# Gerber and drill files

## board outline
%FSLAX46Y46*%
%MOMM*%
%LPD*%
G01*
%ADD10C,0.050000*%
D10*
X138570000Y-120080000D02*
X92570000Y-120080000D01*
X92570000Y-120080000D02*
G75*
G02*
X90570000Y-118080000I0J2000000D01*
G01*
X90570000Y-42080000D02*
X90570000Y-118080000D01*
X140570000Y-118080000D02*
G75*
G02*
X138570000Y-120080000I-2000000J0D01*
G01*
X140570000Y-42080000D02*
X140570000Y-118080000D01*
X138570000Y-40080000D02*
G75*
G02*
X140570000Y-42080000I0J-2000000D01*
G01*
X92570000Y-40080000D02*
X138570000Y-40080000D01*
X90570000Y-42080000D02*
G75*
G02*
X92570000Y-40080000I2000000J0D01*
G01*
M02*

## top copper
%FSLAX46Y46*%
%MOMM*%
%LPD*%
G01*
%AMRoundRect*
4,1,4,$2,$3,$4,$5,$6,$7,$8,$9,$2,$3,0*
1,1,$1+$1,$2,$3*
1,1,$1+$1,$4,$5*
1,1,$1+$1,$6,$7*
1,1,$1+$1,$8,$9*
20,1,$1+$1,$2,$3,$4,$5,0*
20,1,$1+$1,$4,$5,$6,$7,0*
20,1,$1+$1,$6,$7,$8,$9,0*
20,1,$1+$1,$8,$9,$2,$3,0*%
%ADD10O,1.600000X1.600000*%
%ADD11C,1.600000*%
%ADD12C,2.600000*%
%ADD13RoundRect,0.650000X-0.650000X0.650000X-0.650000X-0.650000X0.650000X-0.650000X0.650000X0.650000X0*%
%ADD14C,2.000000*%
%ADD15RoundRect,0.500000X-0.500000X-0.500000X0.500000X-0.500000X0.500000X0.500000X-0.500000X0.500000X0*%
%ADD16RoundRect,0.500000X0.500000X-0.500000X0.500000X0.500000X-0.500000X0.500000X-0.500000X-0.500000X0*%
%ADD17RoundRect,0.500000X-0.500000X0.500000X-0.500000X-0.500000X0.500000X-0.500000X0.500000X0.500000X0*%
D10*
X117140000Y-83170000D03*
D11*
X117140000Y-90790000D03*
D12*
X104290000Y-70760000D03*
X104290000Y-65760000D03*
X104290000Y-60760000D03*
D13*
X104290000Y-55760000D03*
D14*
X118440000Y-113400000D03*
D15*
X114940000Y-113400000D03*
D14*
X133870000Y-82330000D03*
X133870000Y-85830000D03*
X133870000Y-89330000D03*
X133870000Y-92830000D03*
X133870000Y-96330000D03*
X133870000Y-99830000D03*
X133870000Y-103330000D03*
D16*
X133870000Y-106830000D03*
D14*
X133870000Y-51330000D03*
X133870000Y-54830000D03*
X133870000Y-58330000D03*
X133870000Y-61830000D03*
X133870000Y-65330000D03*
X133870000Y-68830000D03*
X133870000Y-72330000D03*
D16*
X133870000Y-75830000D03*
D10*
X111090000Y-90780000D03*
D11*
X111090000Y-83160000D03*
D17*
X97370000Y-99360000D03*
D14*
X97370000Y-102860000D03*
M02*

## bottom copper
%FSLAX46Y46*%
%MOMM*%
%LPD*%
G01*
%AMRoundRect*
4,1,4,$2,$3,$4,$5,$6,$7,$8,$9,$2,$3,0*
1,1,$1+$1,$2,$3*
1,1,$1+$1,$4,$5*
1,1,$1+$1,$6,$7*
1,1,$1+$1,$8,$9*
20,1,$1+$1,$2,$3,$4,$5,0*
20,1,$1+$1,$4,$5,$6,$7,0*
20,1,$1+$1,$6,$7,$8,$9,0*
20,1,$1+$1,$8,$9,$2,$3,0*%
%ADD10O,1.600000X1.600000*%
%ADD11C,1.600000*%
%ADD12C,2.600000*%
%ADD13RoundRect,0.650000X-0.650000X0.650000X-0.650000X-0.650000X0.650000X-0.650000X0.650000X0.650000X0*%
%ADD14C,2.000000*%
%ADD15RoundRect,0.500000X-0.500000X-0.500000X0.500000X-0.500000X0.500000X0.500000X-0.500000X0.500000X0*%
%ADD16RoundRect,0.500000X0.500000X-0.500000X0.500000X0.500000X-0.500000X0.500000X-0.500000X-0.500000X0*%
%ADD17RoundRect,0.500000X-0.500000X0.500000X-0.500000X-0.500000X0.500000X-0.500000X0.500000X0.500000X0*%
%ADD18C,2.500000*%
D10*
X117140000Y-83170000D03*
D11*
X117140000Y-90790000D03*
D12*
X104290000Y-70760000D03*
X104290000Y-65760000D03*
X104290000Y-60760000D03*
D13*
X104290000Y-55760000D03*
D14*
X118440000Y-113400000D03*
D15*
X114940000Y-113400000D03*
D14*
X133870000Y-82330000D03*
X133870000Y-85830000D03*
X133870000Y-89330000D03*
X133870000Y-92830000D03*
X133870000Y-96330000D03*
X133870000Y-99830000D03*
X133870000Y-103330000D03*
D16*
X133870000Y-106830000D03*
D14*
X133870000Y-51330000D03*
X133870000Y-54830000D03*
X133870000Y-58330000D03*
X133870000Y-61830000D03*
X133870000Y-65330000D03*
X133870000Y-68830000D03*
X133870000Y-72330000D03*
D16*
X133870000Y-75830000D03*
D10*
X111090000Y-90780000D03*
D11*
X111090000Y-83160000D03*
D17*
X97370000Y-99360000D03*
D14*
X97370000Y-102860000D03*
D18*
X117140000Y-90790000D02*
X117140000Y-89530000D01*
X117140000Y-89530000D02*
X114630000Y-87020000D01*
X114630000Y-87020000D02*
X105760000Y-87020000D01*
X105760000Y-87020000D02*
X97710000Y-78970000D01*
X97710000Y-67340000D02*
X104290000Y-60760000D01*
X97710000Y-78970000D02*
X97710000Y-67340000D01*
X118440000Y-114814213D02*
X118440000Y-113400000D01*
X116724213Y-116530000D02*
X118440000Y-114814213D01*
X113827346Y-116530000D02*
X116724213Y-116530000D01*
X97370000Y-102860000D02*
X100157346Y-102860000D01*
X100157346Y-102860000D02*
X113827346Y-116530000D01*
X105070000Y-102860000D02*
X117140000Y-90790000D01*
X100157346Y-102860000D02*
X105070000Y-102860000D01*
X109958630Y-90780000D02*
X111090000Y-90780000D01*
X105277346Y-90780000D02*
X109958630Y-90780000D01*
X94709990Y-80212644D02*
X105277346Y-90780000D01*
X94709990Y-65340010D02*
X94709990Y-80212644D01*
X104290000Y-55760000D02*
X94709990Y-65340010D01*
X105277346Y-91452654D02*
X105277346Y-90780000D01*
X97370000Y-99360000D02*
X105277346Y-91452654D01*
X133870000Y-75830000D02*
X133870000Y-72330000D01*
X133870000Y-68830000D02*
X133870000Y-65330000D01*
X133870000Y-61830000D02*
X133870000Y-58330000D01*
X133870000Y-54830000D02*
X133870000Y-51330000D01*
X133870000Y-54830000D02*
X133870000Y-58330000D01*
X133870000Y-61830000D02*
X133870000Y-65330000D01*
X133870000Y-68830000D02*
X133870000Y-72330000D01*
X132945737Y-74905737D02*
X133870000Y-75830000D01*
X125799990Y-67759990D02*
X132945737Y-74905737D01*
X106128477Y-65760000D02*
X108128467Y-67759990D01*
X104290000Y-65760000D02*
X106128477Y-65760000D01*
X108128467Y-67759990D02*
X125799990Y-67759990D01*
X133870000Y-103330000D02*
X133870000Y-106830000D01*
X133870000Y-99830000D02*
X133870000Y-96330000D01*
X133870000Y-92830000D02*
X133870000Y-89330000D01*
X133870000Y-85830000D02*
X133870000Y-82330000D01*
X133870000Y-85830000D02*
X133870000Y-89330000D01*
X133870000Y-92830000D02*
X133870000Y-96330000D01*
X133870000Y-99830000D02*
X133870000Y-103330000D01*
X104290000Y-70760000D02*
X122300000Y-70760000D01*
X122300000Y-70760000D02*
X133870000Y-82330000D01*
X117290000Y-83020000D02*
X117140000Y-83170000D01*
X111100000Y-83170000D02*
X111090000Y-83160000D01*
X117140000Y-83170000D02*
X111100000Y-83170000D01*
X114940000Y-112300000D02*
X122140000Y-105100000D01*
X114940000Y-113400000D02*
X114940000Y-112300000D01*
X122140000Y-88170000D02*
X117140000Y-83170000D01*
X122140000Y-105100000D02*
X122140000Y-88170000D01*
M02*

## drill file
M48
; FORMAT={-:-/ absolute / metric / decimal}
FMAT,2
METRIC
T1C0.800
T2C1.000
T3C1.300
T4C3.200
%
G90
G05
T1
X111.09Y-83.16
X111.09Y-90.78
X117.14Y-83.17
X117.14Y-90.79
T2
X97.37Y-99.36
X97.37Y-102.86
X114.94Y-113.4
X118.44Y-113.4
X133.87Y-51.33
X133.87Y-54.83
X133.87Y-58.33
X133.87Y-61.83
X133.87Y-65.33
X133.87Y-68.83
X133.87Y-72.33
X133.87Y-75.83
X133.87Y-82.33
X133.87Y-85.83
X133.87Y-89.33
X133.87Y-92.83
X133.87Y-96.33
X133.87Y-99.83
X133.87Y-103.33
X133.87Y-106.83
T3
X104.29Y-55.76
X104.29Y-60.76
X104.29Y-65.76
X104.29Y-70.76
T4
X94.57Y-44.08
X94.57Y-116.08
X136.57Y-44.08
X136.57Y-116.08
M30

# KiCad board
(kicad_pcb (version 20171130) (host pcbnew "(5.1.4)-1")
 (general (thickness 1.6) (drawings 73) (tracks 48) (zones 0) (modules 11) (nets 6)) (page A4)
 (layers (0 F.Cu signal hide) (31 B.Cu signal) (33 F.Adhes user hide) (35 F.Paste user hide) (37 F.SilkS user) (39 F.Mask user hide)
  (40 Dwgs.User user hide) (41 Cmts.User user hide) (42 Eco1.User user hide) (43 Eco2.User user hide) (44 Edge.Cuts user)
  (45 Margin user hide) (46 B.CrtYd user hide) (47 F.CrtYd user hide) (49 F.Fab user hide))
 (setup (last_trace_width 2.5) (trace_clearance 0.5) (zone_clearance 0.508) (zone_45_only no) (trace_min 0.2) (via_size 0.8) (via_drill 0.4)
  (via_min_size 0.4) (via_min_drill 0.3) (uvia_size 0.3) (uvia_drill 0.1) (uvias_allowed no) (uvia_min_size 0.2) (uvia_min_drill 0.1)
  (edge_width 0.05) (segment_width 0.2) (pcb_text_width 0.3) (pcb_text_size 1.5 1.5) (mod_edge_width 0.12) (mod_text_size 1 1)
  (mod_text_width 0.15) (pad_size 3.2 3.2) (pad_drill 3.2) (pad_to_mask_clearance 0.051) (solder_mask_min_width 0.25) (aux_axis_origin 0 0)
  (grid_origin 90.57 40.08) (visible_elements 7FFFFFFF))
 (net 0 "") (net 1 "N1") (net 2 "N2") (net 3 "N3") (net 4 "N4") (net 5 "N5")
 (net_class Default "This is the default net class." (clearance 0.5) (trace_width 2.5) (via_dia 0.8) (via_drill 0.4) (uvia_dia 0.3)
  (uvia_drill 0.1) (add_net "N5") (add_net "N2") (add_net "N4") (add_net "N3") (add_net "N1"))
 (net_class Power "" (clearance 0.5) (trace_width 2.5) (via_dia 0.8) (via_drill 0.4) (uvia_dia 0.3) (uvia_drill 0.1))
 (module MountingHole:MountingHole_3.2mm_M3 (layer F.Cu) (at 94.57 116.08)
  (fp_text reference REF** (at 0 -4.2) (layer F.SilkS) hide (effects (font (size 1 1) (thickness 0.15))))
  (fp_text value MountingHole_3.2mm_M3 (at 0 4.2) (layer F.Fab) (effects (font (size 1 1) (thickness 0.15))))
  (pad 1 np_thru_hole circle (at 0 0) (size 3.2 3.2) (drill 3.2) (layers *.Cu *.Mask)))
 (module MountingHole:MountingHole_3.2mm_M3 (layer F.Cu) (at 136.57 116.08)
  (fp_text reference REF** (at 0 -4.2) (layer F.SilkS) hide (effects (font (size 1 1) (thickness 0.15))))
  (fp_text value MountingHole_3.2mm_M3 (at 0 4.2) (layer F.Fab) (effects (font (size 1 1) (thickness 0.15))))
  (pad 1 np_thru_hole circle (at 0 0) (size 3.2 3.2) (drill 3.2) (layers *.Cu *.Mask)))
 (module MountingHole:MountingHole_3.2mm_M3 (layer F.Cu) (at 136.57 44.08)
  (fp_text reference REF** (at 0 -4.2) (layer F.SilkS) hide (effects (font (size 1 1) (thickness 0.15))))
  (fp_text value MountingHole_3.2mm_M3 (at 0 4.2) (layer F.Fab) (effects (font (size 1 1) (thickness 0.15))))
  (pad 1 np_thru_hole circle (at 0 0) (size 3.2 3.2) (drill 3.2) (layers *.Cu *.Mask)))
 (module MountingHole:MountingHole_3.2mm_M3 (layer F.Cu) (at 94.57 44.08)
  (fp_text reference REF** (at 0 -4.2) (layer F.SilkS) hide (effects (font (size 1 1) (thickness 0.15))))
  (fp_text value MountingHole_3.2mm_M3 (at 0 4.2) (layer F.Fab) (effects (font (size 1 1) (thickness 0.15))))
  (pad 1 np_thru_hole circle (at 0 0) (size 3.2 3.2) (drill 3.2) (layers *.Cu *.Mask)))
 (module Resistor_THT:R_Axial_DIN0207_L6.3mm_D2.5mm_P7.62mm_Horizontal (layer F.Cu) (at 117.14 90.79 90)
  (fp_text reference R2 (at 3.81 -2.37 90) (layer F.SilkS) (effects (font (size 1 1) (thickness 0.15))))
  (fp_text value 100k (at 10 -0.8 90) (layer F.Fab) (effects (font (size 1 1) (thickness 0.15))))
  (pad 2 thru_hole oval (at 7.62 0 90) (size 1.6 1.6) (drill 0.8) (layers *.Cu *.Mask) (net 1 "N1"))
  (pad 1 thru_hole circle (at 0 0 90) (size 1.6 1.6) (drill 0.8) (layers *.Cu *.Mask) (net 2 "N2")))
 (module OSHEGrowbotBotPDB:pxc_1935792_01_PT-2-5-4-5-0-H (layer F.Cu) (at 99.79 53.26 270)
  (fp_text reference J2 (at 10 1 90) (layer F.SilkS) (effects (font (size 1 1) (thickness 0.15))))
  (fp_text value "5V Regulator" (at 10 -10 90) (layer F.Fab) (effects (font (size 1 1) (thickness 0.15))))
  (pad 4 thru_hole circle (at 17.5 -4.5 270) (size 2.6 2.6) (drill 1.3) (layers *.Cu *.Mask) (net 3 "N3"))
  (pad 3 thru_hole circle (at 12.5 -4.5 270) (size 2.6 2.6) (drill 1.3) (layers *.Cu *.Mask) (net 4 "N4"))
  (pad 2 thru_hole circle (at 7.5 -4.5 270) (size 2.6 2.6) (drill 1.3) (layers *.Cu *.Mask) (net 2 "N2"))
  (pad 1 thru_hole roundrect (at 2.5 -4.5 270) (size 2.6 2.6) (drill 1.3) (layers *.Cu *.Mask) (roundrect_rratio 0.25) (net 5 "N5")))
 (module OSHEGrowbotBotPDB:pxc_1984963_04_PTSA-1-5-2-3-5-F (layer F.Cu) (at 111.69 118.1)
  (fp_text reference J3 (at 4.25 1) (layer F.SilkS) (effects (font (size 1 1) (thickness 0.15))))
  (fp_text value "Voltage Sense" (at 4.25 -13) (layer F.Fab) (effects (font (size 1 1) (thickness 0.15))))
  (pad 2 thru_hole circle (at 6.75 -4.7) (size 2 2) (drill 1) (layers *.Cu *.Mask) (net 2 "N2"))
  (pad 1 thru_hole roundrect (at 3.25 -4.7) (size 2 2) (drill 1) (layers *.Cu *.Mask) (roundrect_rratio 0.25) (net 1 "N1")))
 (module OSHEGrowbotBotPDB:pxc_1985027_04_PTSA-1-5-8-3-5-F (layer F.Cu) (at 138.57 110.08 90)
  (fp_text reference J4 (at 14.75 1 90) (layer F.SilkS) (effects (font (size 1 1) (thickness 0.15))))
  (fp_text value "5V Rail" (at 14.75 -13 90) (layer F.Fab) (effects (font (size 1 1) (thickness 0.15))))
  (pad 8 thru_hole circle (at 27.75 -4.7 90) (size 2 2) (drill 1) (layers *.Cu *.Mask) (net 3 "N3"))
  (pad 7 thru_hole circle (at 24.25 -4.7 90) (size 2 2) (drill 1) (layers *.Cu *.Mask) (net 3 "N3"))
  (pad 6 thru_hole circle (at 20.75 -4.7 90) (size 2 2) (drill 1) (layers *.Cu *.Mask) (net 3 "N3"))
  (pad 5 thru_hole circle (at 17.25 -4.7 90) (size 2 2) (drill 1) (layers *.Cu *.Mask) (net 3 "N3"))
  (pad 4 thru_hole circle (at 13.75 -4.7 90) (size 2 2) (drill 1) (layers *.Cu *.Mask) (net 3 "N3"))
  (pad 3 thru_hole circle (at 10.25 -4.7 90) (size 2 2) (drill 1) (layers *.Cu *.Mask) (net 3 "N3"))
  (pad 2 thru_hole circle (at 6.75 -4.7 90) (size 2 2) (drill 1) (layers *.Cu *.Mask) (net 3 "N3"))
  (pad 1 thru_hole roundrect (at 3.25 -4.7 90) (size 2 2) (drill 1) (layers *.Cu *.Mask) (roundrect_rratio 0.25) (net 3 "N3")))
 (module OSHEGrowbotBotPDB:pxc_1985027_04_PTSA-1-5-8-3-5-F (layer F.Cu) (at 138.57 79.08 90)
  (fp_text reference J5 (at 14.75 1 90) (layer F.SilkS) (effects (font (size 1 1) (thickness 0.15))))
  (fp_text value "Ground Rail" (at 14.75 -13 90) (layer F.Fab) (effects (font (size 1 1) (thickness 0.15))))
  (pad 8 thru_hole circle (at 27.75 -4.7 90) (size 2 2) (drill 1) (layers *.Cu *.Mask) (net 4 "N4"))
  (pad 7 thru_hole circle (at 24.25 -4.7 90) (size 2 2) (drill 1) (layers *.Cu *.Mask) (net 4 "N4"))
  (pad 6 thru_hole circle (at 20.75 -4.7 90) (size 2 2) (drill 1) (layers *.Cu *.Mask) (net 4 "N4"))
  (pad 5 thru_hole circle (at 17.25 -4.7 90) (size 2 2) (drill 1) (layers *.Cu *.Mask) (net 4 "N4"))
  (pad 4 thru_hole circle (at 13.75 -4.7 90) (size 2 2) (drill 1) (layers *.Cu *.Mask) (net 4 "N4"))
  (pad 3 thru_hole circle (at 10.25 -4.7 90) (size 2 2) (drill 1) (layers *.Cu *.Mask) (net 4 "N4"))
  (pad 2 thru_hole circle (at 6.75 -4.7 90) (size 2 2) (drill 1) (layers *.Cu *.Mask) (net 4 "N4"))
  (pad 1 thru_hole roundrect (at 3.25 -4.7 90) (size 2 2) (drill 1) (layers *.Cu *.Mask) (roundrect_rratio 0.25) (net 4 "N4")))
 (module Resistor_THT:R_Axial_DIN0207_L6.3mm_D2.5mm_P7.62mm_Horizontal (layer F.Cu) (at 111.09 83.16 270)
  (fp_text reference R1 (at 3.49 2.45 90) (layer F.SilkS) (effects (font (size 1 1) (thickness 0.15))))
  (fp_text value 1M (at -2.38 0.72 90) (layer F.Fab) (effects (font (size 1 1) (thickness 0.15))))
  (pad 2 thru_hole oval (at 7.62 0 270) (size 1.6 1.6) (drill 0.8) (layers *.Cu *.Mask) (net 5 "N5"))
  (pad 1 thru_hole circle (at 0 0 270) (size 1.6 1.6) (drill 0.8) (layers *.Cu *.Mask) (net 1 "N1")))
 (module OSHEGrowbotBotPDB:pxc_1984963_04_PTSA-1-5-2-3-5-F (layer F.Cu) (at 92.67 96.11 270)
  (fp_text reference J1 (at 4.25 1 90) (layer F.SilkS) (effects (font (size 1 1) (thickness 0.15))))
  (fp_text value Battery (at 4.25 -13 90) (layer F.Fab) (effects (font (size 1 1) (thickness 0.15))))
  (pad 1 thru_hole roundrect (at 3.25 -4.7 270) (size 2 2) (drill 1) (layers *.Cu *.Mask) (roundrect_rratio 0.25) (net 5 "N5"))
  (pad 2 thru_hole circle (at 6.75 -4.7 270) (size 2 2) (drill 1) (layers *.Cu *.Mask) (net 2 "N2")))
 (gr_line (start 138.57 120.08) (end 92.57 120.08) (layer Edge.Cuts) (width 0.05))
 (gr_arc (start 92.57 118.08) (end 90.57 118.08) (angle -90) (layer Edge.Cuts) (width 0.05))
 (gr_line (start 90.57 42.08) (end 90.57 118.08) (layer Edge.Cuts) (width 0.05))
 (gr_arc (start 138.57 118.08) (end 138.57 120.08) (angle -90) (layer Edge.Cuts) (width 0.05))
 (gr_line (start 140.57 42.08) (end 140.57 118.08) (layer Edge.Cuts) (width 0.05))
 (gr_arc (start 138.57 42.08) (end 140.57 42.08) (angle -90) (layer Edge.Cuts) (width 0.05))
 (gr_line (start 92.57 40.08) (end 138.57 40.08) (layer Edge.Cuts) (width 0.05))
 (gr_arc (start 92.57 42.08) (end 92.57 40.08) (angle -90) (layer Edge.Cuts) (width 0.05))
 (segment (start 117.14 90.79) (end 117.14 89.53) (width 2.5) (layer B.Cu) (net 2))
 (segment (start 117.14 89.53) (end 114.63 87.02) (width 2.5) (layer B.Cu) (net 2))
 (segment (start 114.63 87.02) (end 105.76 87.02) (width 2.5) (layer B.Cu) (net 2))
 (segment (start 105.76 87.02) (end 97.71 78.97) (width 2.5) (layer B.Cu) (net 2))
 (segment (start 97.71 67.34) (end 104.29 60.76) (width 2.5) (layer B.Cu) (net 2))
 (segment (start 97.71 78.97) (end 97.71 67.34) (width 2.5) (layer B.Cu) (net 2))
 (segment (start 118.44 114.814213) (end 118.44 113.4) (width 2.5) (layer B.Cu) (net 2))
 (segment (start 116.724213 116.53) (end 118.44 114.814213) (width 2.5) (layer B.Cu) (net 2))
 (segment (start 113.827346 116.53) (end 116.724213 116.53) (width 2.5) (layer B.Cu) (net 2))
 (segment (start 97.37 102.86) (end 100.157346 102.86) (width 2.5) (layer B.Cu) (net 2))
 (segment (start 100.157346 102.86) (end 113.827346 116.53) (width 2.5) (layer B.Cu) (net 2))
 (segment (start 105.07 102.86) (end 117.14 90.79) (width 2.5) (layer B.Cu) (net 2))
 (segment (start 100.157346 102.86) (end 105.07 102.86) (width 2.5) (layer B.Cu) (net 2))
 (segment (start 109.95863 90.78) (end 111.09 90.78) (width 2.5) (layer B.Cu) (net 5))
 (segment (start 105.277346 90.78) (end 109.95863 90.78) (width 2.5) (layer B.Cu) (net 5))
 (segment (start 94.70999 80.212644) (end 105.277346 90.78) (width 2.5) (layer B.Cu) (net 5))
 (segment (start 94.70999 65.34001) (end 94.70999 80.212644) (width 2.5) (layer B.Cu) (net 5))
 (segment (start 104.29 55.76) (end 94.70999 65.34001) (width 2.5) (layer B.Cu) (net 5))
 (segment (start 105.277346 91.452654) (end 105.277346 90.78) (width 2.5) (layer B.Cu) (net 5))
 (segment (start 97.37 99.36) (end 105.277346 91.452654) (width 2.5) (layer B.Cu) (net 5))
 (segment (start 133.87 75.83) (end 133.87 72.33) (width 2.5) (layer B.Cu) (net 4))
 (segment (start 133.87 68.83) (end 133.87 65.33) (width 2.5) (layer B.Cu) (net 4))
 (segment (start 133.87 61.83) (end 133.87 58.33) (width 2.5) (layer B.Cu) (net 4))
 (segment (start 133.87 54.83) (end 133.87 51.33) (width 2.5) (layer B.Cu) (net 4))
 (segment (start 133.87 54.83) (end 133.87 58.33) (width 2.5) (layer B.Cu) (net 4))
 (segment (start 133.87 61.83) (end 133.87 65.33) (width 2.5) (layer B.Cu) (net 4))
 (segment (start 133.87 68.83) (end 133.87 72.33) (width 2.5) (layer B.Cu) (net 4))
 (segment (start 132.945737 74.905737) (end 133.87 75.83) (width 2.5) (layer B.Cu) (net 4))
 (segment (start 125.79999 67.75999) (end 132.945737 74.905737) (width 2.5) (layer B.Cu) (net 4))
 (segment (start 106.128477 65.76) (end 108.128467 67.75999) (width 2.5) (layer B.Cu) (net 4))
 (segment (start 104.29 65.76) (end 106.128477 65.76) (width 2.5) (layer B.Cu) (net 4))
 (segment (start 108.128467 67.75999) (end 125.79999 67.75999) (width 2.5) (layer B.Cu) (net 4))
 (segment (start 133.87 103.33) (end 133.87 106.83) (width 2.5) (layer B.Cu) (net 3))
 (segment (start 133.87 99.83) (end 133.87 96.33) (width 2.5) (layer B.Cu) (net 3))
 (segment (start 133.87 92.83) (end 133.87 89.33) (width 2.5) (layer B.Cu) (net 3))
 (segment (start 133.87 85.83) (end 133.87 82.33) (width 2.5) (layer B.Cu) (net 3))
 (segment (start 133.87 85.83) (end 133.87 89.33) (width 2.5) (layer B.Cu) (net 3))
 (segment (start 133.87 92.83) (end 133.87 96.33) (width 2.5) (layer B.Cu) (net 3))
 (segment (start 133.87 99.83) (end 133.87 103.33) (width 2.5) (layer B.Cu) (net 3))
 (segment (start 104.29 70.76) (end 122.3 70.76) (width 2.5) (layer B.Cu) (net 3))
 (segment (start 122.3 70.76) (end 133.87 82.33) (width 2.5) (layer B.Cu) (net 3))
 (segment (start 117.29 83.02) (end 117.14 83.17) (width 2.5) (layer B.Cu) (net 1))
 (segment (start 111.1 83.17) (end 111.09 83.16) (width 2.5) (layer B.Cu) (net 1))
 (segment (start 117.14 83.17) (end 111.1 83.17) (width 2.5) (layer B.Cu) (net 1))
 (segment (start 114.94 112.3) (end 122.14 105.1) (width 2.5) (layer B.Cu) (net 1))
 (segment (start 114.94 113.4) (end 114.94 112.3) (width 2.5) (layer B.Cu) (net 1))
 (segment (start 122.14 88.17) (end 117.14 83.17) (width 2.5) (layer B.Cu) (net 1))
 (segment (start 122.14 105.1) (end 122.14 88.17) (width 2.5) (layer B.Cu) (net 1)))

